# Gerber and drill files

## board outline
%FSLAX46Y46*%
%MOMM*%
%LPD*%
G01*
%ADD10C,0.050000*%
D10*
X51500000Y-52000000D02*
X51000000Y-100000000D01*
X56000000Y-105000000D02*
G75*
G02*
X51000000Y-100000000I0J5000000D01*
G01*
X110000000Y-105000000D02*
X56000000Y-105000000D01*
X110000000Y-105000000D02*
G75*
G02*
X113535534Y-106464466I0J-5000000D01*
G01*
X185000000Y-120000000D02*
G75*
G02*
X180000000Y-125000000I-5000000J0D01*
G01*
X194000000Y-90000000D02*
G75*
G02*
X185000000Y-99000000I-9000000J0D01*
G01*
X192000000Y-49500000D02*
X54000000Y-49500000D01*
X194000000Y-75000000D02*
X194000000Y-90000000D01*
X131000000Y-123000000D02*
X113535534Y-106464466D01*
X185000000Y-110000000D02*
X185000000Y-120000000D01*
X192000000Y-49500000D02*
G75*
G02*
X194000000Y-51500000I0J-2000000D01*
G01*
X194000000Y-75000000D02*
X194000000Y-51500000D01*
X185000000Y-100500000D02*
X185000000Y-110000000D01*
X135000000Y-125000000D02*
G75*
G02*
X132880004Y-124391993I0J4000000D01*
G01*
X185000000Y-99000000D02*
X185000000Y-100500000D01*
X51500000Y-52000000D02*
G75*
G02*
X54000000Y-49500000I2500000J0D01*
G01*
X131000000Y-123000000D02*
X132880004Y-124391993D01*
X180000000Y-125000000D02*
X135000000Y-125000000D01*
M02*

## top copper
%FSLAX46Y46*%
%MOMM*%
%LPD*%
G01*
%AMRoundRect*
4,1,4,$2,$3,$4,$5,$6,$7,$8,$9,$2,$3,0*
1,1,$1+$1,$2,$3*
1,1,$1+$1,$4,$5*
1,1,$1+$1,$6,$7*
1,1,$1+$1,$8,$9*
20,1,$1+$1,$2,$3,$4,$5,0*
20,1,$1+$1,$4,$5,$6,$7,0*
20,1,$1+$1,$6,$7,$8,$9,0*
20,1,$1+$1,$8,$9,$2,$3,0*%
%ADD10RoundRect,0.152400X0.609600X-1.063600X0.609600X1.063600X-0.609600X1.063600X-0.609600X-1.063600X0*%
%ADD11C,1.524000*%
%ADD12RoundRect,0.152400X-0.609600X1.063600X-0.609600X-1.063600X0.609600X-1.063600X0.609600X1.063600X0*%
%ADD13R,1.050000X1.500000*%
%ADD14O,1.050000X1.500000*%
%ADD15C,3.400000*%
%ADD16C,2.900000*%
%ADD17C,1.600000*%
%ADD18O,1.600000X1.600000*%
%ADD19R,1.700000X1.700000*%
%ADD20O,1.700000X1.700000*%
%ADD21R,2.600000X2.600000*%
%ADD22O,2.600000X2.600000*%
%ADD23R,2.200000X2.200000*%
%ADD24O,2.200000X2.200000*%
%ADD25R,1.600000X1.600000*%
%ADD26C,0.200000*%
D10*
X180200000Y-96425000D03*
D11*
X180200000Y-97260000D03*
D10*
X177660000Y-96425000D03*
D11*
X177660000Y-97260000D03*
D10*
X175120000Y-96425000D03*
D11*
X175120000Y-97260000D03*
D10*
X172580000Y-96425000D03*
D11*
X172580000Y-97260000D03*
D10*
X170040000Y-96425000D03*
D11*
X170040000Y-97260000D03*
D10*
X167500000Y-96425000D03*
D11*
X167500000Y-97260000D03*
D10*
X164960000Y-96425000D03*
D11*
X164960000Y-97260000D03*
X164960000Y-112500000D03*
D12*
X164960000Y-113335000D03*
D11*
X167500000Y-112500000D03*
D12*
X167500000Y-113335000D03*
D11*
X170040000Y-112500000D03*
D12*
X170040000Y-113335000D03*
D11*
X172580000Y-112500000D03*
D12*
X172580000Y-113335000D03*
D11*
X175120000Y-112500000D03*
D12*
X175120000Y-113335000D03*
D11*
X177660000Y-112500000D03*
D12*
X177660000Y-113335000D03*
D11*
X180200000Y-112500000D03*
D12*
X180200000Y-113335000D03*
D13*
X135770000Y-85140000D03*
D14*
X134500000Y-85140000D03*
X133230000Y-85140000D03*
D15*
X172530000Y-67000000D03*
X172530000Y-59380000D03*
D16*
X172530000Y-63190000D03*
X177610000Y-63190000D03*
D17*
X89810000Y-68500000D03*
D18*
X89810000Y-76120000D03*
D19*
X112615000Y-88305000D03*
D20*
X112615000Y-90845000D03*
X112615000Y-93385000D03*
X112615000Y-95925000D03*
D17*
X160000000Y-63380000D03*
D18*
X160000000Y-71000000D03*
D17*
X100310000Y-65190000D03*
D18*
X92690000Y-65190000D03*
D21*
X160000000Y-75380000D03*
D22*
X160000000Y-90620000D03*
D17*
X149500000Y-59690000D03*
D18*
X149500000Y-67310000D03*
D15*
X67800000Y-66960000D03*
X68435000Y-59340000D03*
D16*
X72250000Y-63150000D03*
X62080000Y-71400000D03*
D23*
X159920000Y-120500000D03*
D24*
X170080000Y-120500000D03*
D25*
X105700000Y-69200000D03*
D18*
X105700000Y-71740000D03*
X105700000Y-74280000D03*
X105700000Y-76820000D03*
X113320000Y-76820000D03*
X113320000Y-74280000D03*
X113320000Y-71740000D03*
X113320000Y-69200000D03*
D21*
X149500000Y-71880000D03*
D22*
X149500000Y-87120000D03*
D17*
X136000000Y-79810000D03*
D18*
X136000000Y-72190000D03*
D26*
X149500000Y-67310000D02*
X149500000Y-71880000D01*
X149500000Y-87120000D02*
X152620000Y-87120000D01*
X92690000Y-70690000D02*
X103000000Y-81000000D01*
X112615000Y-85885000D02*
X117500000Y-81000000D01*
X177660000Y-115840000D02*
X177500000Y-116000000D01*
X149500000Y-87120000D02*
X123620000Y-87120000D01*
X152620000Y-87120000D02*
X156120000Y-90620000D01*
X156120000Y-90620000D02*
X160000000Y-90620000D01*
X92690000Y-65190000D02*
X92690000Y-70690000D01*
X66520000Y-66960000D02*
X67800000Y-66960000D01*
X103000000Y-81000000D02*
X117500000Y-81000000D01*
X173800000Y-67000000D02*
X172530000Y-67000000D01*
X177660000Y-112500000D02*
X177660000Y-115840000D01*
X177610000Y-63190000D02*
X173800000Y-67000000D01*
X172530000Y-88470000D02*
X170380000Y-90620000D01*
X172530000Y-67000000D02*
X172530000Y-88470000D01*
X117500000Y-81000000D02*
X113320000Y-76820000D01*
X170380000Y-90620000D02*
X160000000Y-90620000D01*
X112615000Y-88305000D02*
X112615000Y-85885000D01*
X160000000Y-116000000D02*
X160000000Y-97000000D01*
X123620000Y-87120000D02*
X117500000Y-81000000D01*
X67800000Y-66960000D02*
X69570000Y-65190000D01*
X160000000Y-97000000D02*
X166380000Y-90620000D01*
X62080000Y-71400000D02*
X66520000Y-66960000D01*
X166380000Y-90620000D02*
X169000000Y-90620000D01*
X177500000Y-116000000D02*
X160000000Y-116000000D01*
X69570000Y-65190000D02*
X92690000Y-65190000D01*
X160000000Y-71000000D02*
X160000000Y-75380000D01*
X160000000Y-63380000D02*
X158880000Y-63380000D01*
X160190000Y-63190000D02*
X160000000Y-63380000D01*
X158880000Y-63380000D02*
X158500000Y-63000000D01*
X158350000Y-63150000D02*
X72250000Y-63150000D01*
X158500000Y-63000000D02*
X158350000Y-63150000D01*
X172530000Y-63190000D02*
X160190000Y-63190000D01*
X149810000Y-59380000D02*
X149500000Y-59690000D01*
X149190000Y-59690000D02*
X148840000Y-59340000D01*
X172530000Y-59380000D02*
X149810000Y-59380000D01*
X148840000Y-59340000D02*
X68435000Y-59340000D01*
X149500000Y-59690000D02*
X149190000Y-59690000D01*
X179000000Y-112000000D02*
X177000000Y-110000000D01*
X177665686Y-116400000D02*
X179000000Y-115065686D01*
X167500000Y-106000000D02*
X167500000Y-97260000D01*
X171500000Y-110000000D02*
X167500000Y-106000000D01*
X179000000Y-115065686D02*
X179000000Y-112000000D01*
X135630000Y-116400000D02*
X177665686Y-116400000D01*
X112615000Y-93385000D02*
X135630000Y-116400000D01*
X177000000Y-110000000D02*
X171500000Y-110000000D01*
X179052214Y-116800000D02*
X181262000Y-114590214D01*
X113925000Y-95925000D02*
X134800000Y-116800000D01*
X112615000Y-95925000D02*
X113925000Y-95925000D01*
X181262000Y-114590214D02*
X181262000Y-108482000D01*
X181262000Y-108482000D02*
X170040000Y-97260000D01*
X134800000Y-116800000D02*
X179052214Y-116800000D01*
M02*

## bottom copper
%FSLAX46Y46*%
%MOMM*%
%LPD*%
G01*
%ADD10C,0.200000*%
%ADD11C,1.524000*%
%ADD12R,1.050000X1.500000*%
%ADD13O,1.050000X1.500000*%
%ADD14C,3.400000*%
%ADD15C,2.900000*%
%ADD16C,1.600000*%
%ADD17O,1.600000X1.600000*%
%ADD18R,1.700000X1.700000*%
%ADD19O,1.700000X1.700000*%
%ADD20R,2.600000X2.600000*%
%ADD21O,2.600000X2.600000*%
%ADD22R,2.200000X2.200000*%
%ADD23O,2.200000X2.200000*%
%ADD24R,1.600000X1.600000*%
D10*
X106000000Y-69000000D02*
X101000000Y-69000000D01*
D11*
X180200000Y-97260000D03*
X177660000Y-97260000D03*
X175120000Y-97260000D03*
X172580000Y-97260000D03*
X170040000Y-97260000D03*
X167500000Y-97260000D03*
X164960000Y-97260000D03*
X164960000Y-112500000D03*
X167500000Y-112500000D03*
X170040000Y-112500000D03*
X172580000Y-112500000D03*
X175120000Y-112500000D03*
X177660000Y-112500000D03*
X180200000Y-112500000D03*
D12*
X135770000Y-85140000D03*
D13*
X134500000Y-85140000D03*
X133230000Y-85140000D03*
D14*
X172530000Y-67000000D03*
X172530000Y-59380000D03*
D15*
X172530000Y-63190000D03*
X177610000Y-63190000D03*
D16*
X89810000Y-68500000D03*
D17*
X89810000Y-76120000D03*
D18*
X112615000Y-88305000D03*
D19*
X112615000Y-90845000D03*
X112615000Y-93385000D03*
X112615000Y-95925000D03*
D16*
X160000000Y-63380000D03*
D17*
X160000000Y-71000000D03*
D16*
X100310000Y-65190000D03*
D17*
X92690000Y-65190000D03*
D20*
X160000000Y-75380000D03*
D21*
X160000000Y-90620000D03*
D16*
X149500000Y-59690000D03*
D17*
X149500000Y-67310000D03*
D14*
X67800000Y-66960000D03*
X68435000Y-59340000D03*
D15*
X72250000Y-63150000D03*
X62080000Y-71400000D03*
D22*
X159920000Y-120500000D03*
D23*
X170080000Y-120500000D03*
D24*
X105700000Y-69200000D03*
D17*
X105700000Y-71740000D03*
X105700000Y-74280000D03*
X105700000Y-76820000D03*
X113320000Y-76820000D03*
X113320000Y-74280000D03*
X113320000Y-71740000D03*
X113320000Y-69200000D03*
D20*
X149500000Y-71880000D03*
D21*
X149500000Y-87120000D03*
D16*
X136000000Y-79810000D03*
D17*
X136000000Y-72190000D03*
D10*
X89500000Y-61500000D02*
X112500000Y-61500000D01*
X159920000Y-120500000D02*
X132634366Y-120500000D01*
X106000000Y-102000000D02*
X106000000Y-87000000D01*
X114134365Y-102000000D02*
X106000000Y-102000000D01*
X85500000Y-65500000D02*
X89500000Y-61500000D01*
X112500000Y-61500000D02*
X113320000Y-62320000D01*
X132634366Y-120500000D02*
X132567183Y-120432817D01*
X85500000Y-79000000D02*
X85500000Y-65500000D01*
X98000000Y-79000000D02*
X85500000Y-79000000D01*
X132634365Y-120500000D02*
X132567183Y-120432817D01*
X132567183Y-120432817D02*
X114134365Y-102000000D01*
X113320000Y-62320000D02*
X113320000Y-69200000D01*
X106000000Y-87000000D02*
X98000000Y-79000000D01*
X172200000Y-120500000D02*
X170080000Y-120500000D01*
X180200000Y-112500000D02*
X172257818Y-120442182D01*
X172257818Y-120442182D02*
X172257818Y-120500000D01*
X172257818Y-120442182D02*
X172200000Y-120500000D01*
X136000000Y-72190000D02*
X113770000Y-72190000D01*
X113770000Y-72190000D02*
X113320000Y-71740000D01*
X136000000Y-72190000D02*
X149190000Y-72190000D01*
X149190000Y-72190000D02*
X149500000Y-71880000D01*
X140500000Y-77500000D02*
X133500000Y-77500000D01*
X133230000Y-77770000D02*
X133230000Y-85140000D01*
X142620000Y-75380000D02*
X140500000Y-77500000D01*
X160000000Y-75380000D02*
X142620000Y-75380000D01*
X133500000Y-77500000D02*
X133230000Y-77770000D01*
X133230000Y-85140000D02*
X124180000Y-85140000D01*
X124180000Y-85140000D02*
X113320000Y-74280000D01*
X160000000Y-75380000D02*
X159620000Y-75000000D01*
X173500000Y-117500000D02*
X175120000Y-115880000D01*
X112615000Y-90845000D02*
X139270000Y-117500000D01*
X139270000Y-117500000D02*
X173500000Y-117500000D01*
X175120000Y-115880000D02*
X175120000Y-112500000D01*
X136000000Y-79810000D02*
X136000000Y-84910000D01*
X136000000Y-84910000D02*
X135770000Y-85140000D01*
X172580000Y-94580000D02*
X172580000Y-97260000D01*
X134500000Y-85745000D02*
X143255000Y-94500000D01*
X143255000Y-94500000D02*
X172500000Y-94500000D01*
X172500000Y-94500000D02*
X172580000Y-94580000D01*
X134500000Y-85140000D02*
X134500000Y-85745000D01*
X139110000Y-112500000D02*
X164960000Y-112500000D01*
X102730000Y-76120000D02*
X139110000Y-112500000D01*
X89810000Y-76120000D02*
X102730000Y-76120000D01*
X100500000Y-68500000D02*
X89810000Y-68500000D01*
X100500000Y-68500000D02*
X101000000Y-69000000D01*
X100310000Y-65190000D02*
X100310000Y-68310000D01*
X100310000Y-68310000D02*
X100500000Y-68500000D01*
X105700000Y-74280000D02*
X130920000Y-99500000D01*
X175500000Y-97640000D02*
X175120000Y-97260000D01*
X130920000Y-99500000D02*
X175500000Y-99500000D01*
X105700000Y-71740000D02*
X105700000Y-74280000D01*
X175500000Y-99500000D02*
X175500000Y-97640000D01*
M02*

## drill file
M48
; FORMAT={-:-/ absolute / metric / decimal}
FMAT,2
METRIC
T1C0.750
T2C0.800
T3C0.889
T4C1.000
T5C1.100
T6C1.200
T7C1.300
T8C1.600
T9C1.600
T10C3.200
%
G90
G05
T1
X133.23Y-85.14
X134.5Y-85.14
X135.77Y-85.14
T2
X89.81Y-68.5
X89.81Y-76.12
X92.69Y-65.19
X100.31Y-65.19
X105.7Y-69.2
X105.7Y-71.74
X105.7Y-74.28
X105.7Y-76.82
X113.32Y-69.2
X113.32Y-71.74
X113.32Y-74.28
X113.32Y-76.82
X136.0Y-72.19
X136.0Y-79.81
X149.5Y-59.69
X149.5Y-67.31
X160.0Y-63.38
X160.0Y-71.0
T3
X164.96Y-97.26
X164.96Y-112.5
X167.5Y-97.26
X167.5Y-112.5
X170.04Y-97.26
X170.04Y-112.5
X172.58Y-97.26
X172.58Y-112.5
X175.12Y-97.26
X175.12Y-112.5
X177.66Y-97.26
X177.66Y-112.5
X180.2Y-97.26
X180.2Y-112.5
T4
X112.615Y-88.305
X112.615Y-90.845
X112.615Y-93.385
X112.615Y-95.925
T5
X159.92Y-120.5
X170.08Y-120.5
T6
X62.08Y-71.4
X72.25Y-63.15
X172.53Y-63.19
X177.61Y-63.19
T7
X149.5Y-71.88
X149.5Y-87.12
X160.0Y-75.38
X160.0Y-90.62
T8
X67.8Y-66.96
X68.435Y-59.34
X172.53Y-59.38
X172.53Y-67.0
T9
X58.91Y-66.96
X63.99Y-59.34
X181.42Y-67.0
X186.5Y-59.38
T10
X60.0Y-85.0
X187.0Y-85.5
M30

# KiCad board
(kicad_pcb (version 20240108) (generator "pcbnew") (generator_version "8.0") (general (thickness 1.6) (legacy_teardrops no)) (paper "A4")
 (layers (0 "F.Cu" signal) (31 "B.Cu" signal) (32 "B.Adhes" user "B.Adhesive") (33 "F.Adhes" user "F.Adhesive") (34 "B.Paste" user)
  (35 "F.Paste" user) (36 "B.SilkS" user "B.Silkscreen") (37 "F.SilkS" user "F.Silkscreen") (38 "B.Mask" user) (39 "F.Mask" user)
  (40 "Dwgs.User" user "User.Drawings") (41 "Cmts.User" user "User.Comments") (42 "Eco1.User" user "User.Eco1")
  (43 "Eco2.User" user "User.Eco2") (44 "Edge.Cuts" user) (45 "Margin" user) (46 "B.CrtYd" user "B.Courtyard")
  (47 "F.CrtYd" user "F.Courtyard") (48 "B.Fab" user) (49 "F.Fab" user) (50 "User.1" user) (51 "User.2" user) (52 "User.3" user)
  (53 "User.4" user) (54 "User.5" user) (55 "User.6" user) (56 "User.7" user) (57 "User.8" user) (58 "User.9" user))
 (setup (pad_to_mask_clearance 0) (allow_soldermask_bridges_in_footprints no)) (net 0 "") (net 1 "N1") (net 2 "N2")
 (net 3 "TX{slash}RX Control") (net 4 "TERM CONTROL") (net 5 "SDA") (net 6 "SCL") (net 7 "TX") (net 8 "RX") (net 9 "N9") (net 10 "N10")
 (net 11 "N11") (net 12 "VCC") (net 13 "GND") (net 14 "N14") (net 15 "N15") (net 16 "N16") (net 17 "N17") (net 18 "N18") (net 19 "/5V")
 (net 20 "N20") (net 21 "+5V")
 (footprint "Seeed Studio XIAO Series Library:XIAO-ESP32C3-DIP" (layer "F.Cu") (at 172.58 105 -90)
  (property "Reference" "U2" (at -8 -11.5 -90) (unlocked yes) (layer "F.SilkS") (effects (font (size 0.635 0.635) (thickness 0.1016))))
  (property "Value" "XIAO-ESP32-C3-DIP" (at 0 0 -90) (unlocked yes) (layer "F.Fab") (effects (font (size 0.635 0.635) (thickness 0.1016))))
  (pad "1" smd roundrect (at -8.575 -7.62 90) (size 2.432 1.524) (layers "F.Cu" "F.Mask") (roundrect_rratio 0.1) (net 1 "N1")
   (thermal_bridge_angle 45))
  (pad "1" thru_hole circle (at -7.74 -7.62 90) (size 1.524 1.524) (drill 0.889) (layers "*.Cu" "*.Mask") (remove_unused_layers no)
   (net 1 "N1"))
  (pad "2" smd roundrect (at -8.575 -5.08 90) (size 2.432 1.524) (layers "F.Cu" "F.Mask") (roundrect_rratio 0.1) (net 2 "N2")
   (thermal_bridge_angle 45))
  (pad "2" thru_hole circle (at -7.74 -5.08 90) (size 1.524 1.524) (drill 0.889) (layers "*.Cu" "*.Mask") (remove_unused_layers no)
   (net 2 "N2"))
  (pad "3" smd roundrect (at -8.575 -2.54 90) (size 2.432 1.524) (layers "F.Cu" "F.Mask") (roundrect_rratio 0.1)
   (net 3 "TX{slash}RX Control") (thermal_bridge_angle 45))
  (pad "3" thru_hole circle (at -7.74 -2.54 90) (size 1.524 1.524) (drill 0.889) (layers "*.Cu" "*.Mask") (remove_unused_layers no)
   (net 3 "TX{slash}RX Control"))
  (pad "4" smd roundrect (at -8.575 0 90) (size 2.432 1.524) (layers "F.Cu" "F.Mask") (roundrect_rratio 0.1) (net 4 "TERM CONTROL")
   (thermal_bridge_angle 45))
  (pad "4" thru_hole circle (at -7.74 0 90) (size 1.524 1.524) (drill 0.889) (layers "*.Cu" "*.Mask") (remove_unused_layers no)
   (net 4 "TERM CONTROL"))
  (pad "5" smd roundrect (at -8.575 2.54 90) (size 2.432 1.524) (layers "F.Cu" "F.Mask") (roundrect_rratio 0.1) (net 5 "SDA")
   (thermal_bridge_angle 45))
  (pad "5" thru_hole circle (at -7.74 2.54 90) (size 1.524 1.524) (drill 0.889) (layers "*.Cu" "*.Mask") (remove_unused_layers no)
   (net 5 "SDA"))
  (pad "6" smd roundrect (at -8.575 5.08 90) (size 2.432 1.524) (layers "F.Cu" "F.Mask") (roundrect_rratio 0.1) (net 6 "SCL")
   (thermal_bridge_angle 45))
  (pad "6" thru_hole circle (at -7.74 5.08 90) (size 1.524 1.524) (drill 0.889) (layers "*.Cu" "*.Mask") (remove_unused_layers no)
   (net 6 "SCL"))
  (pad "7" smd roundrect (at -8.575 7.62 90) (size 2.432 1.524) (layers "F.Cu" "F.Mask") (roundrect_rratio 0.1) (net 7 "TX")
   (thermal_bridge_angle 45))
  (pad "7" thru_hole circle (at -7.74 7.62 90) (size 1.524 1.524) (drill 0.889) (layers "*.Cu" "*.Mask") (remove_unused_layers no)
   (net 7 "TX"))
  (pad "8" thru_hole circle (at 7.5 7.62 270) (size 1.524 1.524) (drill 0.889) (layers "*.Cu" "*.Mask") (remove_unused_layers no)
   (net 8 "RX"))
  (pad "8" smd roundrect (at 8.335 7.62 270) (size 2.432 1.524) (layers "F.Cu" "F.Mask") (roundrect_rratio 0.1) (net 8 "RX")
   (thermal_bridge_angle 45))
  (pad "9" thru_hole circle (at 7.5 5.08 270) (size 1.524 1.524) (drill 0.889) (layers "*.Cu" "*.Mask") (remove_unused_layers no)
   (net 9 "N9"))
  (pad "9" smd roundrect (at 8.335 5.08 270) (size 2.432 1.524) (layers "F.Cu" "F.Mask") (roundrect_rratio 0.1) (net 9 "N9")
   (thermal_bridge_angle 45))
  (pad "10" thru_hole circle (at 7.5 2.54 270) (size 1.524 1.524) (drill 0.889) (layers "*.Cu" "*.Mask") (remove_unused_layers no)
   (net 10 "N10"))
  (pad "10" smd roundrect (at 8.335 2.54 270) (size 2.432 1.524) (layers "F.Cu" "F.Mask") (roundrect_rratio 0.1) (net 10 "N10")
   (thermal_bridge_angle 45))
  (pad "11" thru_hole circle (at 7.5 0 270) (size 1.524 1.524) (drill 0.889) (layers "*.Cu" "*.Mask") (remove_unused_layers no)
   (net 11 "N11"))
  (pad "11" smd roundrect (at 8.335 0 270) (size 2.432 1.524) (layers "F.Cu" "F.Mask") (roundrect_rratio 0.1) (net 11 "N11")
   (thermal_bridge_angle 45))
  (pad "12" thru_hole circle (at 7.5 -2.54 270) (size 1.524 1.524) (drill 0.889) (layers "*.Cu" "*.Mask") (remove_unused_layers no)
   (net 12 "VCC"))
  (pad "12" smd roundrect (at 8.335 -2.54 270) (size 2.432 1.524) (layers "F.Cu" "F.Mask") (roundrect_rratio 0.1) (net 12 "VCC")
   (thermal_bridge_angle 45))
  (pad "13" thru_hole circle (at 7.5 -5.08 270) (size 1.524 1.524) (drill 0.889) (layers "*.Cu" "*.Mask") (remove_unused_layers no)
   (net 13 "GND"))
  (pad "13" smd roundrect (at 8.335 -5.08 270) (size 2.432 1.524) (layers "F.Cu" "F.Mask") (roundrect_rratio 0.1) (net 13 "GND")
   (thermal_bridge_angle 45))
  (pad "14" thru_hole circle (at 7.5 -7.62 270) (size 1.524 1.524) (drill 0.889) (layers "*.Cu" "*.Mask") (remove_unused_layers no)
   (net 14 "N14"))
  (pad "14" smd roundrect (at 8.335 -7.62 270) (size 2.432 1.524) (layers "F.Cu" "F.Mask") (roundrect_rratio 0.1) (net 14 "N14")
   (thermal_bridge_angle 45)))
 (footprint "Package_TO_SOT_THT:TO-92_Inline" (layer "F.Cu") (at 135.77 85.14 180)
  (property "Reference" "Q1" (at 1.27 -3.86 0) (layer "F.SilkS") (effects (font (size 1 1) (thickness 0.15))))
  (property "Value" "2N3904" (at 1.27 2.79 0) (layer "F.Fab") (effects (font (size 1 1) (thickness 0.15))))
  (pad "1" thru_hole rect (at 0 0 180) (size 1.05 1.5) (drill 0.75) (layers "*.Cu" "*.Mask") (remove_unused_layers no) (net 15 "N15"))
  (pad "2" thru_hole oval (at 1.27 0 180) (size 1.05 1.5) (drill 0.75) (layers "*.Cu" "*.Mask") (remove_unused_layers no)
   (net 4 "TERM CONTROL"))
  (pad "3" thru_hole oval (at 2.54 0 180) (size 1.05 1.5) (drill 0.75) (layers "*.Cu" "*.Mask") (remove_unused_layers no) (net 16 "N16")))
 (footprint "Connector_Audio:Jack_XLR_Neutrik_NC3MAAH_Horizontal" (layer "F.Cu") (at 172.53 67 90)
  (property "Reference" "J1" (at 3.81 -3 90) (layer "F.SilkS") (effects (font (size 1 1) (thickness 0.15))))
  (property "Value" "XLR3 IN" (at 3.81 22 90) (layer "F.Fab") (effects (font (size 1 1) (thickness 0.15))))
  (pad "" np_thru_hole circle (at 0 8.89 90) (size 1.6 1.6) (drill 1.6) (layers "*.Cu" "*.Mask"))
  (pad "" np_thru_hole circle (at 7.62 13.97 90) (size 1.6 1.6) (drill 1.6) (layers "*.Cu" "*.Mask"))
  (pad "1" thru_hole circle (at 0 0 90) (size 3.4 3.4) (drill 1.6) (layers "*.Cu" "*.Mask") (remove_unused_layers no) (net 13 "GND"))
  (pad "2" thru_hole circle (at 7.62 0 90) (size 3.4 3.4) (drill 1.6) (layers "*.Cu" "*.Mask") (remove_unused_layers no) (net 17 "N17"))
  (pad "3" thru_hole circle (at 3.81 0 90) (size 2.9 2.9) (drill 1.2) (layers "*.Cu" "*.Mask") (remove_unused_layers no) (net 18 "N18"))
  (pad "G" thru_hole circle (at 3.81 5.08 90) (size 2.9 2.9) (drill 1.2) (layers "*.Cu" "*.Mask") (remove_unused_layers no) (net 13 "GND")))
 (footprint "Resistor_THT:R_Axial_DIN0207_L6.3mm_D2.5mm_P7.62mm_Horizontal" (layer "F.Cu") (at 89.81 68.5 -90)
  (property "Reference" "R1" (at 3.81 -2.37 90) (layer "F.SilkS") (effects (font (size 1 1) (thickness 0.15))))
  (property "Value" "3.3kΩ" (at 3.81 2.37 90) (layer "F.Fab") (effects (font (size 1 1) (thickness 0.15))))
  (pad "1" thru_hole circle (at 0 0 270) (size 1.6 1.6) (drill 0.8) (layers "*.Cu" "*.Mask") (remove_unused_layers no) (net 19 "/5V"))
  (pad "2" thru_hole oval (at 7.62 0 270) (size 1.6 1.6) (drill 0.8) (layers "*.Cu" "*.Mask") (remove_unused_layers no) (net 8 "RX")))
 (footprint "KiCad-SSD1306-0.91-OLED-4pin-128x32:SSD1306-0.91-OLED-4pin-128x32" (layer "F.Cu") (at 76.115 86.115)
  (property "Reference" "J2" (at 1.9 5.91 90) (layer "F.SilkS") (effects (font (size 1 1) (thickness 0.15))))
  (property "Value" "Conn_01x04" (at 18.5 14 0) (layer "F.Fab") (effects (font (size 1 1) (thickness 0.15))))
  (pad "1" thru_hole rect (at 36.5 2.19) (size 1.7 1.7) (drill 1) (layers "*.Cu" "*.Mask") (remove_unused_layers no) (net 13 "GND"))
  (pad "2" thru_hole oval (at 36.5 4.73) (size 1.7 1.7) (drill 1) (layers "*.Cu" "*.Mask") (remove_unused_layers no) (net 12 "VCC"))
  (pad "3" thru_hole oval (at 36.5 7.27) (size 1.7 1.7) (drill 1) (layers "*.Cu" "*.Mask") (remove_unused_layers no) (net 6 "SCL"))
  (pad "4" thru_hole oval (at 36.5 9.81) (size 1.7 1.7) (drill 1) (layers "*.Cu" "*.Mask") (remove_unused_layers no) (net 5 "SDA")))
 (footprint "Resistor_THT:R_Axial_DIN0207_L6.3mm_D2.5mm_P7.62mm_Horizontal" (layer "F.Cu") (at 160 63.38 -90)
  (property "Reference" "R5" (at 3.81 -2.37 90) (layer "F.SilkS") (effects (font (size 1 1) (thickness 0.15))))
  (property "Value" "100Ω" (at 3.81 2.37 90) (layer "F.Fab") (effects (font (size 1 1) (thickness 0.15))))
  (pad "1" thru_hole circle (at 0 0 270) (size 1.6 1.6) (drill 0.8) (layers "*.Cu" "*.Mask") (remove_unused_layers no) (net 18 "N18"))
  (pad "2" thru_hole oval (at 7.62 0 270) (size 1.6 1.6) (drill 0.8) (layers "*.Cu" "*.Mask") (remove_unused_layers no) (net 16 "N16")))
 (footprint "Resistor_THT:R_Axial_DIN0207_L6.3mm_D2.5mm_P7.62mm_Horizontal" (layer "F.Cu") (at 100.31 65.19 180)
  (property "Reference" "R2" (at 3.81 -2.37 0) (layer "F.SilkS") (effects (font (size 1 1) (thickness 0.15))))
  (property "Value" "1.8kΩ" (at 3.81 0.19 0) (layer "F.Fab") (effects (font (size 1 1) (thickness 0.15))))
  (pad "1" thru_hole circle (at 0 0 180) (size 1.6 1.6) (drill 0.8) (layers "*.Cu" "*.Mask") (remove_unused_layers no) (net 19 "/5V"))
  (pad "2" thru_hole oval (at 7.62 0 180) (size 1.6 1.6) (drill 0.8) (layers "*.Cu" "*.Mask") (remove_unused_layers no) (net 13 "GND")))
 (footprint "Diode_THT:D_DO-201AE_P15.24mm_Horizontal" (layer "F.Cu") (at 160 75.38 -90)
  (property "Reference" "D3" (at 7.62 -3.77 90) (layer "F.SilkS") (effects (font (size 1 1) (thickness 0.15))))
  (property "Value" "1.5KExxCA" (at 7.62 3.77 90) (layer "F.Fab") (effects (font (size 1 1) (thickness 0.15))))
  (pad "1" thru_hole rect (at 0 0 270) (size 2.6 2.6) (drill 1.3) (layers "*.Cu" "*.Mask") (remove_unused_layers no) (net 16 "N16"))
  (pad "2" thru_hole oval (at 15.24 0 270) (size 2.6 2.6) (drill 1.3) (layers "*.Cu" "*.Mask") (remove_unused_layers no) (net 13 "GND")))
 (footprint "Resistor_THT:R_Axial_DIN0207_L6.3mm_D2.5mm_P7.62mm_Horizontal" (layer "F.Cu") (at 149.5 59.69 -90)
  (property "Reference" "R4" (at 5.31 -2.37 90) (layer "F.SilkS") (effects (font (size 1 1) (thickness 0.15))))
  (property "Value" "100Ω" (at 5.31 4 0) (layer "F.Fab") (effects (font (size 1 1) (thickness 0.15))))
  (pad "1" thru_hole circle (at 0 0 270) (size 1.6 1.6) (drill 0.8) (layers "*.Cu" "*.Mask") (remove_unused_layers no) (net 17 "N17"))
  (pad "2" thru_hole oval (at 7.62 0 270) (size 1.6 1.6) (drill 0.8) (layers "*.Cu" "*.Mask") (remove_unused_layers no) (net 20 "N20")))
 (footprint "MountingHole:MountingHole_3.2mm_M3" (layer "F.Cu") (at 60 85)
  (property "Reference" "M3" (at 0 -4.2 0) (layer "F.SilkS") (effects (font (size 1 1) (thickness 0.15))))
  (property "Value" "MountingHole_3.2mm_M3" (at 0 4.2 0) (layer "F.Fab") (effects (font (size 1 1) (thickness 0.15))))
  (pad "" np_thru_hole circle (at 0 0) (size 3.2 3.2) (drill 3.2) (layers "*.Cu" "*.Mask")))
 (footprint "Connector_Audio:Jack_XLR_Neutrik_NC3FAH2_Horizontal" (layer "F.Cu") (at 67.8 66.96 180)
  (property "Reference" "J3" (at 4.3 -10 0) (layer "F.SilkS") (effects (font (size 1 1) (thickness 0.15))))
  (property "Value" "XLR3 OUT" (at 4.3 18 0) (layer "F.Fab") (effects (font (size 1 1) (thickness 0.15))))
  (pad "" np_thru_hole circle (at 3.81 7.62 180) (size 1.6 1.6) (drill 1.6) (layers "*.Cu" "*.Mask"))
  (pad "" np_thru_hole circle (at 8.89 0 180) (size 1.6 1.6) (drill 1.6) (layers "*.Cu" "*.Mask"))
  (pad "1" thru_hole circle (at 0 0 180) (size 3.4 3.4) (drill 1.6) (layers "*.Cu" "*.Mask") (remove_unused_layers no) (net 13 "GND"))
  (pad "2" thru_hole circle (at -0.635 7.62 180) (size 3.4 3.4) (drill 1.6) (layers "*.Cu" "*.Mask") (remove_unused_layers no)
   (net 17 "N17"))
  (pad "3" thru_hole circle (at -4.45 3.81 180) (size 2.9 2.9) (drill 1.2) (layers "*.Cu" "*.Mask") (remove_unused_layers no) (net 18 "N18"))
  (pad "G" thru_hole circle (at 5.72 -4.44 180) (size 2.9 2.9) (drill 1.2) (layers "*.Cu" "*.Mask") (remove_unused_layers no) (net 13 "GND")))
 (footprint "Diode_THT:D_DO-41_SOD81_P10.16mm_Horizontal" (layer "F.Cu") (at 159.92 120.5)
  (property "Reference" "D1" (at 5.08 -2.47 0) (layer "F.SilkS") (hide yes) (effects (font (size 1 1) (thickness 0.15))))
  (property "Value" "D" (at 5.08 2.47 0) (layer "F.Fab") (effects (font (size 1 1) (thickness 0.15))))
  (pad "1" thru_hole rect (at 0 0) (size 2.2 2.2) (drill 1.1) (layers "*.Cu" "*.Mask") (remove_unused_layers no) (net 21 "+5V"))
  (pad "2" thru_hole oval (at 10.16 0) (size 2.2 2.2) (drill 1.1) (layers "*.Cu" "*.Mask") (remove_unused_layers no) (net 14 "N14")))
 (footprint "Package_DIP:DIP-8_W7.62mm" (layer "F.Cu") (at 105.7 69.2)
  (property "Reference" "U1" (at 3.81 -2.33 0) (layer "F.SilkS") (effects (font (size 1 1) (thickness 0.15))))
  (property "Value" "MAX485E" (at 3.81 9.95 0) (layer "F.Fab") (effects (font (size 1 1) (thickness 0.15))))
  (pad "1" thru_hole rect (at 0 0) (size 1.6 1.6) (drill 0.8) (layers "*.Cu" "*.Mask") (remove_unused_layers no) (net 19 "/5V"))
  (pad "2" thru_hole oval (at 0 2.54) (size 1.6 1.6) (drill 0.8) (layers "*.Cu" "*.Mask") (remove_unused_layers no)
   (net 3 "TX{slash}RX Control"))
  (pad "3" thru_hole oval (at 0 5.08) (size 1.6 1.6) (drill 0.8) (layers "*.Cu" "*.Mask") (remove_unused_layers no)
   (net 3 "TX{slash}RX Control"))
  (pad "4" thru_hole oval (at 0 7.62) (size 1.6 1.6) (drill 0.8) (layers "*.Cu" "*.Mask") (remove_unused_layers no) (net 7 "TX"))
  (pad "5" thru_hole oval (at 7.62 7.62) (size 1.6 1.6) (drill 0.8) (layers "*.Cu" "*.Mask") (remove_unused_layers no) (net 13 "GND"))
  (pad "6" thru_hole oval (at 7.62 5.08) (size 1.6 1.6) (drill 0.8) (layers "*.Cu" "*.Mask") (remove_unused_layers no) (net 16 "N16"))
  (pad "7" thru_hole oval (at 7.62 2.54) (size 1.6 1.6) (drill 0.8) (layers "*.Cu" "*.Mask") (remove_unused_layers no) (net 20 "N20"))
  (pad "8" thru_hole oval (at 7.62 0) (size 1.6 1.6) (drill 0.8) (layers "*.Cu" "*.Mask") (remove_unused_layers no) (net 21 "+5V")))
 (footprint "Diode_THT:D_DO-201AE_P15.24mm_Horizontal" (layer "F.Cu") (at 149.5 71.88 -90)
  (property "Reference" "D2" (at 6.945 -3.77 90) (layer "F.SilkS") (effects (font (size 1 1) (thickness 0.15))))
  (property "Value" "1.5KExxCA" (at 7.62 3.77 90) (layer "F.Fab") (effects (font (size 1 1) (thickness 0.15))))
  (pad "1" thru_hole rect (at 0 0 270) (size 2.6 2.6) (drill 1.3) (layers "*.Cu" "*.Mask") (remove_unused_layers no) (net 20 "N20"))
  (pad "2" thru_hole oval (at 15.24 0 270) (size 2.6 2.6) (drill 1.3) (layers "*.Cu" "*.Mask") (remove_unused_layers no) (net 13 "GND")))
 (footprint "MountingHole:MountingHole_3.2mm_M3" (layer "F.Cu") (at 187 85.5)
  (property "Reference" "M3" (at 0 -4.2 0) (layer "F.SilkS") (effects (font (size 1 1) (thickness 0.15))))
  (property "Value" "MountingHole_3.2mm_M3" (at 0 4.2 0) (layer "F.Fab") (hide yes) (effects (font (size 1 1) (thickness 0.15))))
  (pad "" np_thru_hole circle (at 0 0) (size 3.2 3.2) (drill 3.2) (layers "*.Cu" "*.Mask")))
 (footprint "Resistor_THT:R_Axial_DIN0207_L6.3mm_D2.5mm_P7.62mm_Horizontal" (layer "F.Cu") (at 136 79.81 90)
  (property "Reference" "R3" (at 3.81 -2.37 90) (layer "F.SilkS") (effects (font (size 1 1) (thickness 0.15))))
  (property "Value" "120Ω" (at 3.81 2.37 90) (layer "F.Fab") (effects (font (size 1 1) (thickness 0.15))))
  (pad "1" thru_hole circle (at 0 0 90) (size 1.6 1.6) (drill 0.8) (layers "*.Cu" "*.Mask") (remove_unused_layers no) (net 15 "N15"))
  (pad "2" thru_hole oval (at 7.62 0 90) (size 1.6 1.6) (drill 0.8) (layers "*.Cu" "*.Mask") (remove_unused_layers no) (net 20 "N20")))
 (gr_line (start 106 69) (end 101 69) (stroke (width 0.2) (type default)) (layer "B.Cu") (net 19))
 (gr_line (start 51.5 52) (end 51 100) (stroke (width 0.05) (type default)) (layer "Edge.Cuts"))
 (gr_arc (start 56 105) (mid 52.464466 103.535534) (end 51 100) (stroke (width 0.05) (type default)) (layer "Edge.Cuts"))
 (gr_line (start 110 105) (end 56 105) (stroke (width 0.05) (type default)) (layer "Edge.Cuts"))
 (gr_arc (start 110 105) (mid 111.913417 105.380602) (end 113.535534 106.464466) (stroke (width 0.05) (type default)) (layer "Edge.Cuts"))
 (gr_arc (start 185 120) (mid 183.535534 123.535534) (end 180 125) (stroke (width 0.05) (type default)) (layer "Edge.Cuts"))
 (gr_arc (start 194 90) (mid 191.363961 96.363961) (end 185 99) (stroke (width 0.05) (type default)) (layer "Edge.Cuts"))
 (gr_line (start 192 49.5) (end 54 49.5) (stroke (width 0.05) (type default)) (layer "Edge.Cuts"))
 (gr_line (start 194 75) (end 194 90) (stroke (width 0.05) (type default)) (layer "Edge.Cuts"))
 (gr_line (start 131 123) (end 113.535534 106.464466) (stroke (width 0.05) (type default)) (layer "Edge.Cuts"))
 (gr_line (start 185 110) (end 185 120) (stroke (width 0.05) (type default)) (layer "Edge.Cuts"))
 (gr_arc (start 192 49.5) (mid 193.414214 50.085786) (end 194 51.5) (stroke (width 0.05) (type default)) (layer "Edge.Cuts"))
 (gr_line (start 194 75) (end 194 51.5) (stroke (width 0.05) (type default)) (layer "Edge.Cuts"))
 (gr_line (start 185 100.5) (end 185 110) (stroke (width 0.05) (type default)) (layer "Edge.Cuts"))
 (gr_arc (start 135 125) (mid 133.89727 124.844995) (end 132.880004 124.391993) (stroke (width 0.05) (type default)) (layer "Edge.Cuts"))
 (gr_line (start 185 99) (end 185 100.5) (stroke (width 0.05) (type default)) (layer "Edge.Cuts"))
 (gr_arc (start 51.5 52) (mid 52.232233 50.232233) (end 54 49.5) (stroke (width 0.05) (type default)) (layer "Edge.Cuts"))
 (gr_line (start 131 123) (end 132.880004 124.391993) (stroke (width 0.05) (type default)) (layer "Edge.Cuts"))
 (gr_line (start 180 125) (end 135 125) (stroke (width 0.05) (type default)) (layer "Edge.Cuts"))
 (segment (start 89.5 61.5) (end 112.5 61.5) (width 0.2) (layer "B.Cu") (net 21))
 (segment (start 159.92 120.5) (end 132.634366 120.5) (width 0.2) (layer "B.Cu") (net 21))
 (segment (start 106 102) (end 106 87) (width 0.2) (layer "B.Cu") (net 21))
 (segment (start 114.134365 102) (end 106 102) (width 0.2) (layer "B.Cu") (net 21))
 (segment (start 85.5 65.5) (end 89.5 61.5) (width 0.2) (layer "B.Cu") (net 21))
 (segment (start 112.5 61.5) (end 113.32 62.32) (width 0.2) (layer "B.Cu") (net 21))
 (segment (start 132.634366 120.5) (end 132.567183 120.432817) (width 0.2) (layer "B.Cu") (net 21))
 (segment (start 85.5 79) (end 85.5 65.5) (width 0.2) (layer "B.Cu") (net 21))
 (segment (start 98 79) (end 85.5 79) (width 0.2) (layer "B.Cu") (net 21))
 (segment (start 132.634365 120.5) (end 132.567183 120.432817) (width 0.2) (layer "B.Cu") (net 21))
 (segment (start 132.567183 120.432817) (end 114.134365 102) (width 0.2) (layer "B.Cu") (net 21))
 (segment (start 113.32 62.32) (end 113.32 69.2) (width 0.2) (layer "B.Cu") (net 21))
 (segment (start 106 87) (end 98 79) (width 0.2) (layer "B.Cu") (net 21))
 (segment (start 172.2 120.5) (end 170.08 120.5) (width 0.2) (layer "B.Cu") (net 14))
 (segment (start 180.2 112.5) (end 172.257818 120.442182) (width 0.2) (layer "B.Cu") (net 14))
 (segment (start 172.257818 120.442182) (end 172.257818 120.5) (width 0.2) (layer "B.Cu") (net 14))
 (segment (start 172.257818 120.442182) (end 172.2 120.5) (width 0.2) (layer "B.Cu") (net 14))
 (segment (start 149.5 67.31) (end 149.5 71.88) (width 0.2) (layer "F.Cu") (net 20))
 (segment (start 136 72.19) (end 113.77 72.19) (width 0.2) (layer "B.Cu") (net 20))
 (segment (start 113.77 72.19) (end 113.32 71.74) (width 0.2) (layer "B.Cu") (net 20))
 (segment (start 136 72.19) (end 149.19 72.19) (width 0.2) (layer "B.Cu") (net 20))
 (segment (start 149.19 72.19) (end 149.5 71.88) (width 0.2) (layer "B.Cu") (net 20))
 (segment (start 149.5 87.12) (end 152.62 87.12) (width 0.2) (layer "F.Cu") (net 13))
 (segment (start 92.69 70.69) (end 103 81) (width 0.2) (layer "F.Cu") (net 13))
 (segment (start 112.615 85.885) (end 117.5 81) (width 0.2) (layer "F.Cu") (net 13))
 (segment (start 177.66 115.84) (end 177.5 116) (width 0.2) (layer "F.Cu") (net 13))
 (segment (start 149.5 87.12) (end 123.62 87.12) (width 0.2) (layer "F.Cu") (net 13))
 (segment (start 152.62 87.12) (end 156.12 90.62) (width 0.2) (layer "F.Cu") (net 13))
 (segment (start 156.12 90.62) (end 160 90.62) (width 0.2) (layer "F.Cu") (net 13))
 (segment (start 92.69 65.19) (end 92.69 70.69) (width 0.2) (layer "F.Cu") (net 13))
 (segment (start 66.52 66.96) (end 67.8 66.96) (width 0.2) (layer "F.Cu") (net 13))
 (segment (start 103 81) (end 117.5 81) (width 0.2) (layer "F.Cu") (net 13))
 (segment (start 173.8 67) (end 172.53 67) (width 0.2) (layer "F.Cu") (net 13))
 (segment (start 177.66 112.5) (end 177.66 115.84) (width 0.2) (layer "F.Cu") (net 13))
 (segment (start 177.61 63.19) (end 173.8 67) (width 0.2) (layer "F.Cu") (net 13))
 (segment (start 172.53 88.47) (end 170.38 90.62) (width 0.2) (layer "F.Cu") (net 13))
 (segment (start 172.53 67) (end 172.53 88.47) (width 0.2) (layer "F.Cu") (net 13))
 (segment (start 117.5 81) (end 113.32 76.82) (width 0.2) (layer "F.Cu") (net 13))
 (segment (start 170.38 90.62) (end 160 90.62) (width 0.2) (layer "F.Cu") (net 13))
 (segment (start 112.615 88.305) (end 112.615 85.885) (width 0.2) (layer "F.Cu") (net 13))
 (segment (start 160 116) (end 160 97) (width 0.2) (layer "F.Cu") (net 13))
 (segment (start 123.62 87.12) (end 117.5 81) (width 0.2) (layer "F.Cu") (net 13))
 (segment (start 67.8 66.96) (end 69.57 65.19) (width 0.2) (layer "F.Cu") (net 13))
 (segment (start 160 97) (end 166.38 90.62) (width 0.2) (layer "F.Cu") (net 13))
 (segment (start 62.08 71.4) (end 66.52 66.96) (width 0.2) (layer "F.Cu") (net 13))
 (segment (start 166.38 90.62) (end 169 90.62) (width 0.2) (layer "F.Cu") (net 13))
 (segment (start 177.5 116) (end 160 116) (width 0.2) (layer "F.Cu") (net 13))
 (segment (start 69.57 65.19) (end 92.69 65.19) (width 0.2) (layer "F.Cu") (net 13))
 (segment (start 160 71) (end 160 75.38) (width 0.2) (layer "F.Cu") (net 16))
 (segment (start 140.5 77.5) (end 133.5 77.5) (width 0.2) (layer "B.Cu") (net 16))
 (segment (start 133.23 77.77) (end 133.23 85.14) (width 0.2) (layer "B.Cu") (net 16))
 (segment (start 142.62 75.38) (end 140.5 77.5) (width 0.2) (layer "B.Cu") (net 16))
 (segment (start 160 75.38) (end 142.62 75.38) (width 0.2) (layer "B.Cu") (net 16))
 (segment (start 133.5 77.5) (end 133.23 77.77) (width 0.2) (layer "B.Cu") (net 16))
 (segment (start 133.23 85.14) (end 124.18 85.14) (width 0.2) (layer "B.Cu") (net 16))
 (segment (start 124.18 85.14) (end 113.32 74.28) (width 0.2) (layer "B.Cu") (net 16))
 (segment (start 160 75.38) (end 159.62 75) (width 0.2) (layer "B.Cu") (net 16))
 (segment (start 160 63.38) (end 158.88 63.38) (width 0.2) (layer "F.Cu") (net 18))
 (segment (start 160.19 63.19) (end 160 63.38) (width 0.2) (layer "F.Cu") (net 18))
 (segment (start 158.88 63.38) (end 158.5 63) (width 0.2) (layer "F.Cu") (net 18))
 (segment (start 158.35 63.15) (end 72.25 63.15) (width 0.2) (layer "F.Cu") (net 18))
 (segment (start 158.5 63) (end 158.35 63.15) (width 0.2) (layer "F.Cu") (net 18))
 (segment (start 172.53 63.19) (end 160.19 63.19) (width 0.2) (layer "F.Cu") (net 18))
 (segment (start 149.81 59.38) (end 149.5 59.69) (width 0.2) (layer "F.Cu") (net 17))
 (segment (start 149.19 59.69) (end 148.84 59.34) (width 0.2) (layer "F.Cu") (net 17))
 (segment (start 172.53 59.38) (end 149.81 59.38) (width 0.2) (layer "F.Cu") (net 17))
 (segment (start 148.84 59.34) (end 68.435 59.34) (width 0.2) (layer "F.Cu") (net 17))
 (segment (start 149.5 59.69) (end 149.19 59.69) (width 0.2) (layer "F.Cu") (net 17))
 (segment (start 173.5 117.5) (end 175.12 115.88) (width 0.2) (layer "B.Cu") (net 12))
 (segment (start 112.615 90.845) (end 139.27 117.5) (width 0.2) (layer "B.Cu") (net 12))
 (segment (start 139.27 117.5) (end 173.5 117.5) (width 0.2) (layer "B.Cu") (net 12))
 (segment (start 175.12 115.88) (end 175.12 112.5) (width 0.2) (layer "B.Cu") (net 12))
 (segment (start 179 112) (end 177 110) (width 0.2) (layer "F.Cu") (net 6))
 (segment (start 177.665686 116.4) (end 179 115.065686) (width 0.2) (layer "F.Cu") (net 6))
 (segment (start 167.5 106) (end 167.5 97.26) (width 0.2) (layer "F.Cu") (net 6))
 (segment (start 171.5 110) (end 167.5 106) (width 0.2) (layer "F.Cu") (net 6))
 (segment (start 179 115.065686) (end 179 112) (width 0.2) (layer "F.Cu") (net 6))
 (segment (start 135.63 116.4) (end 177.665686 116.4) (width 0.2) (layer "F.Cu") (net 6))
 (segment (start 112.615 93.385) (end 135.63 116.4) (width 0.2) (layer "F.Cu") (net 6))
 (segment (start 177 110) (end 171.5 110) (width 0.2) (layer "F.Cu") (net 6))
 (segment (start 179.052214 116.8) (end 181.262 114.590214) (width 0.2) (layer "F.Cu") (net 5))
 (segment (start 113.925 95.925) (end 134.8 116.8) (width 0.2) (layer "F.Cu") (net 5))
 (segment (start 112.615 95.925) (end 113.925 95.925) (width 0.2) (layer "F.Cu") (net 5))
 (segment (start 181.262 114.590214) (end 181.262 108.482) (width 0.2) (layer "F.Cu") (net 5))
 (segment (start 181.262 108.482) (end 170.04 97.26) (width 0.2) (layer "F.Cu") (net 5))
 (segment (start 134.8 116.8) (end 179.052214 116.8) (width 0.2) (layer "F.Cu") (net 5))
 (segment (start 136 79.81) (end 136 84.91) (width 0.2) (layer "B.Cu") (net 15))
 (segment (start 136 84.91) (end 135.77 85.14) (width 0.2) (layer "B.Cu") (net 15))
 (segment (start 172.58 94.58) (end 172.58 97.26) (width 0.2) (layer "B.Cu") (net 4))
 (segment (start 134.5 85.745) (end 143.255 94.5) (width 0.2) (layer "B.Cu") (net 4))
 (segment (start 143.255 94.5) (end 172.5 94.5) (width 0.2) (layer "B.Cu") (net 4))
 (segment (start 172.5 94.5) (end 172.58 94.58) (width 0.2) (layer "B.Cu") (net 4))
 (segment (start 134.5 85.14) (end 134.5 85.745) (width 0.2) (layer "B.Cu") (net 4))
 (segment (start 139.11 112.5) (end 164.96 112.5) (width 0.2) (layer "B.Cu") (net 8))
 (segment (start 102.73 76.12) (end 139.11 112.5) (width 0.2) (layer "B.Cu") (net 8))
 (segment (start 89.81 76.12) (end 102.73 76.12) (width 0.2) (layer "B.Cu") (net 8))
 (segment (start 100.5 68.5) (end 89.81 68.5) (width 0.2) (layer "B.Cu") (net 19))
 (segment (start 100.5 68.5) (end 101 69) (width 0.2) (layer "B.Cu") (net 19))
 (segment (start 100.31 65.19) (end 100.31 68.31) (width 0.2) (layer "B.Cu") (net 19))
 (segment (start 100.31 68.31) (end 100.5 68.5) (width 0.2) (layer "B.Cu") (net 19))
 (segment (start 105.7 74.28) (end 130.92 99.5) (width 0.2) (layer "B.Cu") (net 3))
 (segment (start 175.5 97.64) (end 175.12 97.26) (width 0.2) (layer "B.Cu") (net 3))
 (segment (start 130.92 99.5) (end 175.5 99.5) (width 0.2) (layer "B.Cu") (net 3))
 (segment (start 105.7 71.74) (end 105.7 74.28) (width 0.2) (layer "B.Cu") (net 3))
 (segment (start 175.5 99.5) (end 175.5 97.64) (width 0.2) (layer "B.Cu") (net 3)))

